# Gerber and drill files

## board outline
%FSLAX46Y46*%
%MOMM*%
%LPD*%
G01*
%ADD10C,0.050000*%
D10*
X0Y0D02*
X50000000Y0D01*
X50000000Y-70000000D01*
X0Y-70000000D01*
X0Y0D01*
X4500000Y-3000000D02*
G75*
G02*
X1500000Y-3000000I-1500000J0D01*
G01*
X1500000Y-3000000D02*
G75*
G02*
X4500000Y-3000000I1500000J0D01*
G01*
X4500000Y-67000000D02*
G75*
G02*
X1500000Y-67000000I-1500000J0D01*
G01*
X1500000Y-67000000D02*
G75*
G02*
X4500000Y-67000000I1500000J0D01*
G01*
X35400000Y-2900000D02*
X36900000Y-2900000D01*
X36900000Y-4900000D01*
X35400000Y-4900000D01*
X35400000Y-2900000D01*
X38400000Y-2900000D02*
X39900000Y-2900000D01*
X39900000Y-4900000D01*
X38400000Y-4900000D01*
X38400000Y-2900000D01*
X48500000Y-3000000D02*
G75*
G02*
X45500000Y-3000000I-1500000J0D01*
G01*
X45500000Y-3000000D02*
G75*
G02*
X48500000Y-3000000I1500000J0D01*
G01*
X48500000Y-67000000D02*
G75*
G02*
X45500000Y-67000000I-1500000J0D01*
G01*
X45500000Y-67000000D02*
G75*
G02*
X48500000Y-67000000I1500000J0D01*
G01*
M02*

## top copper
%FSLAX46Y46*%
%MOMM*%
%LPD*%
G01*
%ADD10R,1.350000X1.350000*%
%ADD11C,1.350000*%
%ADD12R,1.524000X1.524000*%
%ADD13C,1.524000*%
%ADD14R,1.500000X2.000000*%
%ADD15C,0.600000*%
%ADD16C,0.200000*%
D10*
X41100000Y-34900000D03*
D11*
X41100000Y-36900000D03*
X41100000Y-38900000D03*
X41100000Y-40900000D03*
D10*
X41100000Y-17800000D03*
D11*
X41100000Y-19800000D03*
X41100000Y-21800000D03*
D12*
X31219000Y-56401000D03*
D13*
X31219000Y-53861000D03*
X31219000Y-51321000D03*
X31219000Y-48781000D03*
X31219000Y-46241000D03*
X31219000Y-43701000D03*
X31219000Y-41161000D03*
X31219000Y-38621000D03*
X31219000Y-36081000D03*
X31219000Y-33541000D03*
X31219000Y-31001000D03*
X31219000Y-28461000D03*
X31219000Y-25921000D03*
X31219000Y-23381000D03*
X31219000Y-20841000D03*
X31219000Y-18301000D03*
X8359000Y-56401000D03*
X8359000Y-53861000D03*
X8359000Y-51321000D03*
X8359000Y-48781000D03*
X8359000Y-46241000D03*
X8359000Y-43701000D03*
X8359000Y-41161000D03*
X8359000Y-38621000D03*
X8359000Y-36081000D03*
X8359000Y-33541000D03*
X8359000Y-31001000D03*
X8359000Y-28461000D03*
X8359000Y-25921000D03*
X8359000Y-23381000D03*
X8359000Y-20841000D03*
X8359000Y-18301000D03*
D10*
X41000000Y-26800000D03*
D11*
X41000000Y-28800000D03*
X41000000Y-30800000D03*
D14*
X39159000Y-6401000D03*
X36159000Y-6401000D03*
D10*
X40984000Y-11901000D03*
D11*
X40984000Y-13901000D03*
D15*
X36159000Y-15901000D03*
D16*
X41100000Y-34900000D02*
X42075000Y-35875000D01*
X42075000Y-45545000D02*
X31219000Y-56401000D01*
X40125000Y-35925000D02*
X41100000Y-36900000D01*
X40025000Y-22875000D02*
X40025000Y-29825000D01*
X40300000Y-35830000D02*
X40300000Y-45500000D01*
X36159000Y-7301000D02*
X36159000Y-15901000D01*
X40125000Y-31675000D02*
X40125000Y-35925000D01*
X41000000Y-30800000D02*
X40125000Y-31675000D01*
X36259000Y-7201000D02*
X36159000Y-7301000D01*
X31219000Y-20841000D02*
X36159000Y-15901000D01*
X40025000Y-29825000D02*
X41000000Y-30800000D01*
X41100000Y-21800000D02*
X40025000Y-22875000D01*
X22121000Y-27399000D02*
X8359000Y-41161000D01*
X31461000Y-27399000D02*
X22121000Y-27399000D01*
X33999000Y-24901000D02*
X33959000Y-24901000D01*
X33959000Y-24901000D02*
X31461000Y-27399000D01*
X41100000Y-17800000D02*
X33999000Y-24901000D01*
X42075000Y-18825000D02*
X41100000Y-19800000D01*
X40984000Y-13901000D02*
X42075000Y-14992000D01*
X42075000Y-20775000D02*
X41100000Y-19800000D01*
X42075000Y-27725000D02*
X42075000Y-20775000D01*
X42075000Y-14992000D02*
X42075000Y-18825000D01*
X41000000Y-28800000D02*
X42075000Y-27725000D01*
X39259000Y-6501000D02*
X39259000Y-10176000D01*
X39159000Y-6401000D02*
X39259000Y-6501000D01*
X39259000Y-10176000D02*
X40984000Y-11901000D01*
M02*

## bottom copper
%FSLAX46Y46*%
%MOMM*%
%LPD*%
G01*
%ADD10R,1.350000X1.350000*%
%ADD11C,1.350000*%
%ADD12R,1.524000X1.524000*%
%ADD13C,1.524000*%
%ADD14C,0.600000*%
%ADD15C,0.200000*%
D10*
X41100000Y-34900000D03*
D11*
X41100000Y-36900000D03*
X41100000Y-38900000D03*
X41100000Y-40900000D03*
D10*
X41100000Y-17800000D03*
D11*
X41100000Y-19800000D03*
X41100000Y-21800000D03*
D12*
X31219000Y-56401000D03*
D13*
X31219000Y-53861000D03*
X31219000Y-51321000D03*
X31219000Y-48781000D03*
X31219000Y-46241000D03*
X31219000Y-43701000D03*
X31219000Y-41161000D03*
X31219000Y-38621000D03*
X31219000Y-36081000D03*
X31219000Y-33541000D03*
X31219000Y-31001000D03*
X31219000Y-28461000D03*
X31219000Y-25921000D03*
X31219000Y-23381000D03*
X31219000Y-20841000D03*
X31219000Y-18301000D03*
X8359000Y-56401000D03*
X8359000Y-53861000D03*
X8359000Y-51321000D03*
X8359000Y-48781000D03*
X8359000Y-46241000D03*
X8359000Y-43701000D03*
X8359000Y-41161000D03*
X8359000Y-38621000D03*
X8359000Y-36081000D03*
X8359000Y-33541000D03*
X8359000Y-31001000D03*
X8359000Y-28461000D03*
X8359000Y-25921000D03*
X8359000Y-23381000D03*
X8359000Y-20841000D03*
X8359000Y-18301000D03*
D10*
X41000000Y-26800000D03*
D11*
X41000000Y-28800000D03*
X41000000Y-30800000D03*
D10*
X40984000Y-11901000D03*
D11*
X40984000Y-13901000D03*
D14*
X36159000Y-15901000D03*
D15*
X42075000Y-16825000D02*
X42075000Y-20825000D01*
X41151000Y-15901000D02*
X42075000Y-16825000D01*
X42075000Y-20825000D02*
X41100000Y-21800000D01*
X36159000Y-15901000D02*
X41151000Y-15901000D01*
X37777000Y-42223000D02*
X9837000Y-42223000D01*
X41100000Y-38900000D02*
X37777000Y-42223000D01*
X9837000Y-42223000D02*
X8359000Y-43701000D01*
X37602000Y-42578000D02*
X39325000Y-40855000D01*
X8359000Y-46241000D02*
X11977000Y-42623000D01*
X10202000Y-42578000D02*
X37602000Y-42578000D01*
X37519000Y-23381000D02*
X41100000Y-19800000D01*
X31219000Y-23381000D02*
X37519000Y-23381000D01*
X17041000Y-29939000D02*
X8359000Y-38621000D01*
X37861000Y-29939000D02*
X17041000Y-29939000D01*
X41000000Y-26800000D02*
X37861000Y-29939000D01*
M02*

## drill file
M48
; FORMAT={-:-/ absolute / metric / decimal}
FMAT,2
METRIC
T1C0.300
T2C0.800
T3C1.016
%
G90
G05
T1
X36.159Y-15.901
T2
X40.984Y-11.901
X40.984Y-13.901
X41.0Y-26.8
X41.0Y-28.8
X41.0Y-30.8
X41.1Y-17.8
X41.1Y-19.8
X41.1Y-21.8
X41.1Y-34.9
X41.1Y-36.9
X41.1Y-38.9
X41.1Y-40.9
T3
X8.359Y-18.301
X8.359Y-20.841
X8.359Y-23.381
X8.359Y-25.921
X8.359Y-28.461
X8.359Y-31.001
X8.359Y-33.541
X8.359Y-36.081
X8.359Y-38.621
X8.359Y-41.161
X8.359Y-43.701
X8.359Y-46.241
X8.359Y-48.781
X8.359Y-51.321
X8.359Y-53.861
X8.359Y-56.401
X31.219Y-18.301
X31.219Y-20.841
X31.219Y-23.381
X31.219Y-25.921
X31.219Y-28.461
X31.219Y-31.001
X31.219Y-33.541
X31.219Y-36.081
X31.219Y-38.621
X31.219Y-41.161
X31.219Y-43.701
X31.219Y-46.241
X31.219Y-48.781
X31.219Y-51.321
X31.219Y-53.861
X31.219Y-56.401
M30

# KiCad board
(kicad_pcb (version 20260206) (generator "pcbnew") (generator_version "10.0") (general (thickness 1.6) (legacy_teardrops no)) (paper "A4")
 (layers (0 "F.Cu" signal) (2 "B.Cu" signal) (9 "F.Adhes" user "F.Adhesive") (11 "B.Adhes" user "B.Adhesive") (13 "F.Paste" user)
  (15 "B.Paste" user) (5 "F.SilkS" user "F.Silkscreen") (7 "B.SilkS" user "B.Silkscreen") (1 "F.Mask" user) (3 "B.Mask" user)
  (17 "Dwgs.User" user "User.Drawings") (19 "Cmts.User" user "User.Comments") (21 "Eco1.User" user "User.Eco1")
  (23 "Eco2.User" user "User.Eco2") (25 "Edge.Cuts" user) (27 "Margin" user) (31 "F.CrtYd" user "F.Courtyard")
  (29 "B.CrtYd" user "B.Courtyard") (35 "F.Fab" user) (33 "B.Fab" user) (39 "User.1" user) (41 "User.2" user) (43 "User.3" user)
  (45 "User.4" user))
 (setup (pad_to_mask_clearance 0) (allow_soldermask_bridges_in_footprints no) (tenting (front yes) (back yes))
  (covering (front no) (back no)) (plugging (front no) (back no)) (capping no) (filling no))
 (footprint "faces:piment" (layer "F.Cu") (at 41.9 60.5)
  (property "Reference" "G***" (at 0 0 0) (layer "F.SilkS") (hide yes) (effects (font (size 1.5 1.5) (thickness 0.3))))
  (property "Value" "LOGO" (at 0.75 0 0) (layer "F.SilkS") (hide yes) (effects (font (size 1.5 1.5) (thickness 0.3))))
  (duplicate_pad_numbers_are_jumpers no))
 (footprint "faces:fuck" (layer "F.Cu") (at 21.816165 37.3 90)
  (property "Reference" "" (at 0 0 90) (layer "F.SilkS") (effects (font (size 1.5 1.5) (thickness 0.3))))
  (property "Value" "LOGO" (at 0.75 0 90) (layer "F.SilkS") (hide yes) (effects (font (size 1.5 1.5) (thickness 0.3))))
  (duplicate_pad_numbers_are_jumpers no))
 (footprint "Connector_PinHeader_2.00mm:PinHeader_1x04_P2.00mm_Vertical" (layer "F.Cu") (at 41.1 34.9)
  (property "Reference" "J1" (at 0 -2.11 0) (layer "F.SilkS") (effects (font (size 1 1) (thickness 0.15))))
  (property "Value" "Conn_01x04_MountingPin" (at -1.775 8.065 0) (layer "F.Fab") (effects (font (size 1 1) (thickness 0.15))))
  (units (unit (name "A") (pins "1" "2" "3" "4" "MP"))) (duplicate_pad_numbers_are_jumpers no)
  (pad "1" thru_hole rect (at 0 0) (size 1.35 1.35) (drill 0.8) (layers "*.Cu" "*.Mask") (remove_unused_layers no) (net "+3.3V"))
  (pad "2" thru_hole circle (at 0 2) (size 1.35 1.35) (drill 0.8) (layers "*.Cu" "*.Mask") (remove_unused_layers no) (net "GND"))
  (pad "3" thru_hole circle (at 0 4) (size 1.35 1.35) (drill 0.8) (layers "*.Cu" "*.Mask") (remove_unused_layers no) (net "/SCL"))
  (pad "4" thru_hole circle (at 0 6) (size 1.35 1.35) (drill 0.8) (layers "*.Cu" "*.Mask") (remove_unused_layers no) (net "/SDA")))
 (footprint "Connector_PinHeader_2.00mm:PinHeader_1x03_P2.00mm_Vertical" (layer "F.Cu") (at 41.1 17.8)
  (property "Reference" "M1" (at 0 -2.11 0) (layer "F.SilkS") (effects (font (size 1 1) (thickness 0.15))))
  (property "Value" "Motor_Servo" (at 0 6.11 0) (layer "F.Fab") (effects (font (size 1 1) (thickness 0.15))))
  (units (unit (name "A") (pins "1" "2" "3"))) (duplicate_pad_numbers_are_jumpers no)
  (pad "1" thru_hole rect (at 0 0) (size 1.35 1.35) (drill 0.8) (layers "*.Cu" "*.Mask") (remove_unused_layers no) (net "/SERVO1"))
  (pad "2" thru_hole circle (at 0 2) (size 1.35 1.35) (drill 0.8) (layers "*.Cu" "*.Mask") (remove_unused_layers no) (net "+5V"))
  (pad "3" thru_hole circle (at 0 4) (size 1.35 1.35) (drill 0.8) (layers "*.Cu" "*.Mask") (remove_unused_layers no) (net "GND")))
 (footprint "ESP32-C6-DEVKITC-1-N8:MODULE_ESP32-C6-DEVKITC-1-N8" (layer "F.Cu") (at 19.789 32.076 180)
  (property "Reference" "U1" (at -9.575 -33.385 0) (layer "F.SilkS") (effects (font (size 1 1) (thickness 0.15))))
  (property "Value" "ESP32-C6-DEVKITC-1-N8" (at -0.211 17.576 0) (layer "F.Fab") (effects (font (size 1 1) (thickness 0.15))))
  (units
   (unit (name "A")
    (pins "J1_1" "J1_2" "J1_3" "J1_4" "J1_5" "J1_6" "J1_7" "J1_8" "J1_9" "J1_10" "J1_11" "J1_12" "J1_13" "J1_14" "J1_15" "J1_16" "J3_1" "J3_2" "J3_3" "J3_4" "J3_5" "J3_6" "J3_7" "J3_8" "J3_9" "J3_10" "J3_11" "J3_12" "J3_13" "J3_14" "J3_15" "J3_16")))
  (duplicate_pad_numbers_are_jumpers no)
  (pad "J1_1" thru_hole rect (at -11.43 -24.325 180) (size 1.524 1.524) (drill 1.016) (layers "*.Cu" "*.Mask") (remove_unused_layers no)
   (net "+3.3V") (solder_mask_margin 0.102))
  (pad "J1_2" thru_hole circle (at -11.43 -21.785 180) (size 1.524 1.524) (drill 1.016) (layers "*.Cu" "*.Mask") (remove_unused_layers no)
   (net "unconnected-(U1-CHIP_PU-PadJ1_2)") (solder_mask_margin 0.102))
  (pad "J1_3" thru_hole circle (at -11.43 -19.245 180) (size 1.524 1.524) (drill 1.016) (layers "*.Cu" "*.Mask") (remove_unused_layers no)
   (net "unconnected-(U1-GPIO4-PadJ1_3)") (solder_mask_margin 0.102))
  (pad "J1_4" thru_hole circle (at -11.43 -16.705 180) (size 1.524 1.524) (drill 1.016) (layers "*.Cu" "*.Mask") (remove_unused_layers no)
   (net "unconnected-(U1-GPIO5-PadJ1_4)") (solder_mask_margin 0.102))
  (pad "J1_5" thru_hole circle (at -11.43 -14.165 180) (size 1.524 1.524) (drill 1.016) (layers "*.Cu" "*.Mask") (remove_unused_layers no)
   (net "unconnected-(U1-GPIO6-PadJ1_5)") (solder_mask_margin 0.102))
  (pad "J1_6" thru_hole circle (at -11.43 -11.625 180) (size 1.524 1.524) (drill 1.016) (layers "*.Cu" "*.Mask") (remove_unused_layers no)
   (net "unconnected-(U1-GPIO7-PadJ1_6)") (solder_mask_margin 0.102))
  (pad "J1_7" thru_hole circle (at -11.43 -9.085 180) (size 1.524 1.524) (drill 1.016) (layers "*.Cu" "*.Mask") (remove_unused_layers no)
   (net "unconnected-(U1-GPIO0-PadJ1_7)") (solder_mask_margin 0.102))
  (pad "J1_8" thru_hole circle (at -11.43 -6.545 180) (size 1.524 1.524) (drill 1.016) (layers "*.Cu" "*.Mask") (remove_unused_layers no)
   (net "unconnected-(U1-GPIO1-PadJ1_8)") (solder_mask_margin 0.102))
  (pad "J1_9" thru_hole circle (at -11.43 -4.005 180) (size 1.524 1.524) (drill 1.016) (layers "*.Cu" "*.Mask") (remove_unused_layers no)
   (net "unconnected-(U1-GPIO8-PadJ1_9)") (solder_mask_margin 0.102))
  (pad "J1_10" thru_hole circle (at -11.43 -1.465 180) (size 1.524 1.524) (drill 1.016) (layers "*.Cu" "*.Mask") (remove_unused_layers no)
   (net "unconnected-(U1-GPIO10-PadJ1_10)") (solder_mask_margin 0.102))
  (pad "J1_11" thru_hole circle (at -11.43 1.075 180) (size 1.524 1.524) (drill 1.016) (layers "*.Cu" "*.Mask") (remove_unused_layers no)
   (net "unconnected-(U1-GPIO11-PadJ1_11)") (solder_mask_margin 0.102))
  (pad "J1_12" thru_hole circle (at -11.43 3.615 180) (size 1.524 1.524) (drill 1.016) (layers "*.Cu" "*.Mask") (remove_unused_layers no)
   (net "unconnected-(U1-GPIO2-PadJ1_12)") (solder_mask_margin 0.102))
  (pad "J1_13" thru_hole circle (at -11.43 6.155 180) (size 1.524 1.524) (drill 1.016) (layers "*.Cu" "*.Mask") (remove_unused_layers no)
   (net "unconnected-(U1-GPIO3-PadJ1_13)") (solder_mask_margin 0.102))
  (pad "J1_14" thru_hole circle (at -11.43 8.695 180) (size 1.524 1.524) (drill 1.016) (layers "*.Cu" "*.Mask") (remove_unused_layers no)
   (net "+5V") (solder_mask_margin 0.102))
  (pad "J1_15" thru_hole circle (at -11.43 11.235 180) (size 1.524 1.524) (drill 1.016) (layers "*.Cu" "*.Mask") (remove_unused_layers no)
   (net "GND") (solder_mask_margin 0.102))
  (pad "J1_16" thru_hole circle (at -11.43 13.775 180) (size 1.524 1.524) (drill 1.016) (layers "*.Cu" "*.Mask") (remove_unused_layers no)
   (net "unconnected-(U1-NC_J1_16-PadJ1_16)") (solder_mask_margin 0.102))
  (pad "J3_1" thru_hole circle (at 11.43 -24.325 180) (size 1.524 1.524) (drill 1.016) (layers "*.Cu" "*.Mask") (remove_unused_layers no)
   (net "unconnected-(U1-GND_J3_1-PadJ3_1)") (solder_mask_margin 0.102))
  (pad "J3_2" thru_hole circle (at 11.43 -21.785 180) (size 1.524 1.524) (drill 1.016) (layers "*.Cu" "*.Mask") (remove_unused_layers no)
   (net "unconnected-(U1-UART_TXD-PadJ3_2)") (solder_mask_margin 0.102))
  (pad "J3_3" thru_hole circle (at 11.43 -19.245 180) (size 1.524 1.524) (drill 1.016) (layers "*.Cu" "*.Mask") (remove_unused_layers no)
   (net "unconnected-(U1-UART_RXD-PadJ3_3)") (solder_mask_margin 0.102))
  (pad "J3_4" thru_hole circle (at 11.43 -16.705 180) (size 1.524 1.524) (drill 1.016) (layers "*.Cu" "*.Mask") (remove_unused_layers no)
   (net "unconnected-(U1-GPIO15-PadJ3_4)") (solder_mask_margin 0.102))
  (pad "J3_5" thru_hole circle (at 11.43 -14.165 180) (size 1.524 1.524) (drill 1.016) (layers "*.Cu" "*.Mask") (remove_unused_layers no)
   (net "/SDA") (solder_mask_margin 0.102))
  (pad "J3_6" thru_hole circle (at 11.43 -11.625 180) (size 1.524 1.524) (drill 1.016) (layers "*.Cu" "*.Mask") (remove_unused_layers no)
   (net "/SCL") (solder_mask_margin 0.102))
  (pad "J3_7" thru_hole circle (at 11.43 -9.085 180) (size 1.524 1.524) (drill 1.016) (layers "*.Cu" "*.Mask") (remove_unused_layers no)
   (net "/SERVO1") (solder_mask_margin 0.102))
  (pad "J3_8" thru_hole circle (at 11.43 -6.545 180) (size 1.524 1.524) (drill 1.016) (layers "*.Cu" "*.Mask") (remove_unused_layers no)
   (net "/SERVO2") (solder_mask_margin 0.102))
  (pad "J3_9" thru_hole circle (at 11.43 -4.005 180) (size 1.524 1.524) (drill 1.016) (layers "*.Cu" "*.Mask") (remove_unused_layers no)
   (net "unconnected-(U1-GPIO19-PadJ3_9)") (solder_mask_margin 0.102))
  (pad "J3_10" thru_hole circle (at 11.43 -1.465 180) (size 1.524 1.524) (drill 1.016) (layers "*.Cu" "*.Mask") (remove_unused_layers no)
   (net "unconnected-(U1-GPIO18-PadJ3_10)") (solder_mask_margin 0.102))
  (pad "J3_11" thru_hole circle (at 11.43 1.075 180) (size 1.524 1.524) (drill 1.016) (layers "*.Cu" "*.Mask") (remove_unused_layers no)
   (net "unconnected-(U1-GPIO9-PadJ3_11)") (solder_mask_margin 0.102))
  (pad "J3_12" thru_hole circle (at 11.43 3.615 180) (size 1.524 1.524) (drill 1.016) (layers "*.Cu" "*.Mask") (remove_unused_layers no)
   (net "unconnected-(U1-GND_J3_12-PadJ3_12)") (solder_mask_margin 0.102))
  (pad "J3_13" thru_hole circle (at 11.43 6.155 180) (size 1.524 1.524) (drill 1.016) (layers "*.Cu" "*.Mask") (remove_unused_layers no)
   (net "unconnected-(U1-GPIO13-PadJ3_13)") (solder_mask_margin 0.102))
  (pad "J3_14" thru_hole circle (at 11.43 8.695 180) (size 1.524 1.524) (drill 1.016) (layers "*.Cu" "*.Mask") (remove_unused_layers no)
   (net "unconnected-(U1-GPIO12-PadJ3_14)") (solder_mask_margin 0.102))
  (pad "J3_15" thru_hole circle (at 11.43 11.235 180) (size 1.524 1.524) (drill 1.016) (layers "*.Cu" "*.Mask") (remove_unused_layers no)
   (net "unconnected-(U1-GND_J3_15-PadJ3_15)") (solder_mask_margin 0.102))
  (pad "J3_16" thru_hole circle (at 11.43 13.775 180) (size 1.524 1.524) (drill 1.016) (layers "*.Cu" "*.Mask") (remove_unused_layers no)
   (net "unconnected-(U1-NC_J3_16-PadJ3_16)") (solder_mask_margin 0.102)))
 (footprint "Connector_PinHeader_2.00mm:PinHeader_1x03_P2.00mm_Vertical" (layer "F.Cu") (at 41 26.8)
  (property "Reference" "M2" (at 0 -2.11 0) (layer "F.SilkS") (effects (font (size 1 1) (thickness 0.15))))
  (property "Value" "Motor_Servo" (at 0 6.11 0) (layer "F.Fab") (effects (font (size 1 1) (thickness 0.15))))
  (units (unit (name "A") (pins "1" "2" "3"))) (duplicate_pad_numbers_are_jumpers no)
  (pad "1" thru_hole rect (at 0 0) (size 1.35 1.35) (drill 0.8) (layers "*.Cu" "*.Mask") (remove_unused_layers no) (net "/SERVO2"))
  (pad "2" thru_hole circle (at 0 2) (size 1.35 1.35) (drill 0.8) (layers "*.Cu" "*.Mask") (remove_unused_layers no) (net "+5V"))
  (pad "3" thru_hole circle (at 0 4) (size 1.35 1.35) (drill 0.8) (layers "*.Cu" "*.Mask") (remove_unused_layers no) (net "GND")))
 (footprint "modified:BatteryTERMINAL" (layer "F.Cu") (at 37.659 6.401 -90)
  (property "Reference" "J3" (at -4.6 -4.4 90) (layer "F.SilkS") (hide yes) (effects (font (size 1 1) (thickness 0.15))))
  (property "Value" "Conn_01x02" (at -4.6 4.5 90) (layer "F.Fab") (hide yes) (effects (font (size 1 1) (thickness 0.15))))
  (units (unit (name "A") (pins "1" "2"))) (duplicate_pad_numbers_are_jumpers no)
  (pad "1" smd rect (at 0 -1.5 270) (size 2 1.5) (layers "F.Cu" "F.Mask" "F.Paste") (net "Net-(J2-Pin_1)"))
  (pad "2" smd rect (at 0 1.5 270) (size 2 1.5) (layers "F.Cu" "F.Mask" "F.Paste") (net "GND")))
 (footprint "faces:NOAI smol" (layer "F.Cu") (at 44.463826 47.802621)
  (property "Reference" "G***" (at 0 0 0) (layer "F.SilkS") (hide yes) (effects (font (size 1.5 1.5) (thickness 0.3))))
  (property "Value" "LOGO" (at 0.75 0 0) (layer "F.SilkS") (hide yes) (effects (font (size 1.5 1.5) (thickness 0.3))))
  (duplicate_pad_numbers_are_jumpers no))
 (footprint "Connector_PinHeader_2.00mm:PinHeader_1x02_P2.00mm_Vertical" (layer "F.Cu") (at 40.984 11.901)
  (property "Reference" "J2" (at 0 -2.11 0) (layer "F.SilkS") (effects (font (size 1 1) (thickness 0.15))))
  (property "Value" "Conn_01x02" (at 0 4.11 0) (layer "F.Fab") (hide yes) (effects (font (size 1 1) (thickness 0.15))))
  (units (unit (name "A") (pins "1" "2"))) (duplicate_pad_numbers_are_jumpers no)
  (pad "1" thru_hole rect (at 0 0) (size 1.35 1.35) (drill 0.8) (layers "*.Cu" "*.Mask") (remove_unused_layers no) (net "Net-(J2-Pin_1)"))
  (pad "2" thru_hole circle (at 0 2) (size 1.35 1.35) (drill 0.8) (layers "*.Cu" "*.Mask") (remove_unused_layers no) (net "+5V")))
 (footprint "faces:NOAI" (layer "B.Cu") (at 23.3 36.7 180)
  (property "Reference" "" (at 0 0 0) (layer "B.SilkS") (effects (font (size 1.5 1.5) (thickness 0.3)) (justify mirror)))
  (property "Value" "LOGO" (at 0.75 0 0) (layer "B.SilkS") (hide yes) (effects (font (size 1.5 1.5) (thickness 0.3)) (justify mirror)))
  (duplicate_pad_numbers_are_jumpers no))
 (gr_rect (start 0 0) (end 50 70) (stroke (width 0.05) (type solid)) (fill no) (layer "Edge.Cuts"))
 (gr_circle (center 3 3) (end 4.5 3) (stroke (width 0.05) (type solid)) (fill no) (layer "Edge.Cuts"))
 (gr_circle (center 3 67) (end 4.5 67) (stroke (width 0.05) (type solid)) (fill no) (layer "Edge.Cuts"))
 (gr_rect (start 35.4 2.9) (end 36.9 4.9) (stroke (width 0.05) (type solid)) (fill no) (layer "Edge.Cuts"))
 (gr_rect (start 38.4 2.9) (end 39.9 4.9) (stroke (width 0.05) (type solid)) (fill no) (layer "Edge.Cuts"))
 (gr_circle (center 47 3) (end 48.5 3) (stroke (width 0.05) (type solid)) (fill no) (layer "Edge.Cuts"))
 (gr_circle (center 47 67) (end 48.5 67) (stroke (width 0.05) (type solid)) (fill no) (layer "Edge.Cuts"))
 (segment (start 41.1 34.9) (end 42.075 35.875) (width 0.2) (layer "F.Cu") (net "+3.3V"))
 (segment (start 42.075 45.545) (end 31.219 56.401) (width 0.2) (layer "F.Cu") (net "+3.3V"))
 (segment (start 40.125 35.925) (end 41.1 36.9) (width 0.2) (layer "F.Cu") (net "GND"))
 (segment (start 40.025 22.875) (end 40.025 29.825) (width 0.2) (layer "F.Cu") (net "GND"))
 (segment (start 40.3 35.83) (end 40.3 45.5) (width 0.2) (layer "F.Cu") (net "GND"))
 (segment (start 36.159 7.301) (end 36.159 15.901) (width 0.2) (layer "F.Cu") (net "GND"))
 (segment (start 40.125 31.675) (end 40.125 35.925) (width 0.2) (layer "F.Cu") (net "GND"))
 (segment (start 41 30.8) (end 40.125 31.675) (width 0.2) (layer "F.Cu") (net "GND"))
 (segment (start 36.259 7.201) (end 36.159 7.301) (width 0.2) (layer "F.Cu") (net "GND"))
 (segment (start 31.219 20.841) (end 36.159 15.901) (width 0.2) (layer "F.Cu") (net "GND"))
 (segment (start 40.025 29.825) (end 41 30.8) (width 0.2) (layer "F.Cu") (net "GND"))
 (segment (start 41.1 21.8) (end 40.025 22.875) (width 0.2) (layer "F.Cu") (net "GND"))
 (via (at 36.159 15.901) (size 0.6) (drill 0.3) (layers "F.Cu" "B.Cu") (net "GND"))
 (segment (start 42.075 16.825) (end 42.075 20.825) (width 0.2) (layer "B.Cu") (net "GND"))
 (segment (start 41.151 15.901) (end 42.075 16.825) (width 0.2) (layer "B.Cu") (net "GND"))
 (segment (start 42.075 20.825) (end 41.1 21.8) (width 0.2) (layer "B.Cu") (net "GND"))
 (segment (start 36.159 15.901) (end 41.151 15.901) (width 0.2) (layer "B.Cu") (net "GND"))
 (segment (start 37.777 42.223) (end 9.837 42.223) (width 0.2) (layer "B.Cu") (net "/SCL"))
 (segment (start 41.1 38.9) (end 37.777 42.223) (width 0.2) (layer "B.Cu") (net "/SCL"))
 (segment (start 9.837 42.223) (end 8.359 43.701) (width 0.2) (layer "B.Cu") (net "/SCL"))
 (segment (start 37.602 42.578) (end 39.325 40.855) (width 0.2) (layer "B.Cu") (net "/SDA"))
 (segment (start 8.359 46.241) (end 11.977 42.623) (width 0.2) (layer "B.Cu") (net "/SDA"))
 (segment (start 10.202 42.578) (end 37.602 42.578) (width 0.2) (layer "B.Cu") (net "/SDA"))
 (segment (start 22.121 27.399) (end 8.359 41.161) (width 0.2) (layer "F.Cu") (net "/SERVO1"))
 (segment (start 31.461 27.399) (end 22.121 27.399) (width 0.2) (layer "F.Cu") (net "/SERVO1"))
 (segment (start 33.999 24.901) (end 33.959 24.901) (width 0.2) (layer "F.Cu") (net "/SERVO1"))
 (segment (start 33.959 24.901) (end 31.461 27.399) (width 0.2) (layer "F.Cu") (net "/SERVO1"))
 (segment (start 41.1 17.8) (end 33.999 24.901) (width 0.2) (layer "F.Cu") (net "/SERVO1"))
 (segment (start 42.075 18.825) (end 41.1 19.8) (width 0.2) (layer "F.Cu") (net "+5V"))
 (segment (start 40.984 13.901) (end 42.075 14.992) (width 0.2) (layer "F.Cu") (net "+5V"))
 (segment (start 42.075 20.775) (end 41.1 19.8) (width 0.2) (layer "F.Cu") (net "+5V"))
 (segment (start 42.075 27.725) (end 42.075 20.775) (width 0.2) (layer "F.Cu") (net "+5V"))
 (segment (start 42.075 14.992) (end 42.075 18.825) (width 0.2) (layer "F.Cu") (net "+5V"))
 (segment (start 41 28.8) (end 42.075 27.725) (width 0.2) (layer "F.Cu") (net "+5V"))
 (segment (start 37.519 23.381) (end 41.1 19.8) (width 0.2) (layer "B.Cu") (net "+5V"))
 (segment (start 31.219 23.381) (end 37.519 23.381) (width 0.2) (layer "B.Cu") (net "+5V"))
 (segment (start 17.041 29.939) (end 8.359 38.621) (width 0.2) (layer "B.Cu") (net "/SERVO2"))
 (segment (start 37.861 29.939) (end 17.041 29.939) (width 0.2) (layer "B.Cu") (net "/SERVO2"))
 (segment (start 41 26.8) (end 37.861 29.939) (width 0.2) (layer "B.Cu") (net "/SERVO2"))
 (segment (start 39.259 6.501) (end 39.259 10.176) (width 0.2) (layer "F.Cu") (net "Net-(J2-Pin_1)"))
 (segment (start 39.159 6.401) (end 39.259 6.501) (width 0.2) (layer "F.Cu") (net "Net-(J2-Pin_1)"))
 (segment (start 39.259 10.176) (end 40.984 11.901) (width 0.2) (layer "F.Cu") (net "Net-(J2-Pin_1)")))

